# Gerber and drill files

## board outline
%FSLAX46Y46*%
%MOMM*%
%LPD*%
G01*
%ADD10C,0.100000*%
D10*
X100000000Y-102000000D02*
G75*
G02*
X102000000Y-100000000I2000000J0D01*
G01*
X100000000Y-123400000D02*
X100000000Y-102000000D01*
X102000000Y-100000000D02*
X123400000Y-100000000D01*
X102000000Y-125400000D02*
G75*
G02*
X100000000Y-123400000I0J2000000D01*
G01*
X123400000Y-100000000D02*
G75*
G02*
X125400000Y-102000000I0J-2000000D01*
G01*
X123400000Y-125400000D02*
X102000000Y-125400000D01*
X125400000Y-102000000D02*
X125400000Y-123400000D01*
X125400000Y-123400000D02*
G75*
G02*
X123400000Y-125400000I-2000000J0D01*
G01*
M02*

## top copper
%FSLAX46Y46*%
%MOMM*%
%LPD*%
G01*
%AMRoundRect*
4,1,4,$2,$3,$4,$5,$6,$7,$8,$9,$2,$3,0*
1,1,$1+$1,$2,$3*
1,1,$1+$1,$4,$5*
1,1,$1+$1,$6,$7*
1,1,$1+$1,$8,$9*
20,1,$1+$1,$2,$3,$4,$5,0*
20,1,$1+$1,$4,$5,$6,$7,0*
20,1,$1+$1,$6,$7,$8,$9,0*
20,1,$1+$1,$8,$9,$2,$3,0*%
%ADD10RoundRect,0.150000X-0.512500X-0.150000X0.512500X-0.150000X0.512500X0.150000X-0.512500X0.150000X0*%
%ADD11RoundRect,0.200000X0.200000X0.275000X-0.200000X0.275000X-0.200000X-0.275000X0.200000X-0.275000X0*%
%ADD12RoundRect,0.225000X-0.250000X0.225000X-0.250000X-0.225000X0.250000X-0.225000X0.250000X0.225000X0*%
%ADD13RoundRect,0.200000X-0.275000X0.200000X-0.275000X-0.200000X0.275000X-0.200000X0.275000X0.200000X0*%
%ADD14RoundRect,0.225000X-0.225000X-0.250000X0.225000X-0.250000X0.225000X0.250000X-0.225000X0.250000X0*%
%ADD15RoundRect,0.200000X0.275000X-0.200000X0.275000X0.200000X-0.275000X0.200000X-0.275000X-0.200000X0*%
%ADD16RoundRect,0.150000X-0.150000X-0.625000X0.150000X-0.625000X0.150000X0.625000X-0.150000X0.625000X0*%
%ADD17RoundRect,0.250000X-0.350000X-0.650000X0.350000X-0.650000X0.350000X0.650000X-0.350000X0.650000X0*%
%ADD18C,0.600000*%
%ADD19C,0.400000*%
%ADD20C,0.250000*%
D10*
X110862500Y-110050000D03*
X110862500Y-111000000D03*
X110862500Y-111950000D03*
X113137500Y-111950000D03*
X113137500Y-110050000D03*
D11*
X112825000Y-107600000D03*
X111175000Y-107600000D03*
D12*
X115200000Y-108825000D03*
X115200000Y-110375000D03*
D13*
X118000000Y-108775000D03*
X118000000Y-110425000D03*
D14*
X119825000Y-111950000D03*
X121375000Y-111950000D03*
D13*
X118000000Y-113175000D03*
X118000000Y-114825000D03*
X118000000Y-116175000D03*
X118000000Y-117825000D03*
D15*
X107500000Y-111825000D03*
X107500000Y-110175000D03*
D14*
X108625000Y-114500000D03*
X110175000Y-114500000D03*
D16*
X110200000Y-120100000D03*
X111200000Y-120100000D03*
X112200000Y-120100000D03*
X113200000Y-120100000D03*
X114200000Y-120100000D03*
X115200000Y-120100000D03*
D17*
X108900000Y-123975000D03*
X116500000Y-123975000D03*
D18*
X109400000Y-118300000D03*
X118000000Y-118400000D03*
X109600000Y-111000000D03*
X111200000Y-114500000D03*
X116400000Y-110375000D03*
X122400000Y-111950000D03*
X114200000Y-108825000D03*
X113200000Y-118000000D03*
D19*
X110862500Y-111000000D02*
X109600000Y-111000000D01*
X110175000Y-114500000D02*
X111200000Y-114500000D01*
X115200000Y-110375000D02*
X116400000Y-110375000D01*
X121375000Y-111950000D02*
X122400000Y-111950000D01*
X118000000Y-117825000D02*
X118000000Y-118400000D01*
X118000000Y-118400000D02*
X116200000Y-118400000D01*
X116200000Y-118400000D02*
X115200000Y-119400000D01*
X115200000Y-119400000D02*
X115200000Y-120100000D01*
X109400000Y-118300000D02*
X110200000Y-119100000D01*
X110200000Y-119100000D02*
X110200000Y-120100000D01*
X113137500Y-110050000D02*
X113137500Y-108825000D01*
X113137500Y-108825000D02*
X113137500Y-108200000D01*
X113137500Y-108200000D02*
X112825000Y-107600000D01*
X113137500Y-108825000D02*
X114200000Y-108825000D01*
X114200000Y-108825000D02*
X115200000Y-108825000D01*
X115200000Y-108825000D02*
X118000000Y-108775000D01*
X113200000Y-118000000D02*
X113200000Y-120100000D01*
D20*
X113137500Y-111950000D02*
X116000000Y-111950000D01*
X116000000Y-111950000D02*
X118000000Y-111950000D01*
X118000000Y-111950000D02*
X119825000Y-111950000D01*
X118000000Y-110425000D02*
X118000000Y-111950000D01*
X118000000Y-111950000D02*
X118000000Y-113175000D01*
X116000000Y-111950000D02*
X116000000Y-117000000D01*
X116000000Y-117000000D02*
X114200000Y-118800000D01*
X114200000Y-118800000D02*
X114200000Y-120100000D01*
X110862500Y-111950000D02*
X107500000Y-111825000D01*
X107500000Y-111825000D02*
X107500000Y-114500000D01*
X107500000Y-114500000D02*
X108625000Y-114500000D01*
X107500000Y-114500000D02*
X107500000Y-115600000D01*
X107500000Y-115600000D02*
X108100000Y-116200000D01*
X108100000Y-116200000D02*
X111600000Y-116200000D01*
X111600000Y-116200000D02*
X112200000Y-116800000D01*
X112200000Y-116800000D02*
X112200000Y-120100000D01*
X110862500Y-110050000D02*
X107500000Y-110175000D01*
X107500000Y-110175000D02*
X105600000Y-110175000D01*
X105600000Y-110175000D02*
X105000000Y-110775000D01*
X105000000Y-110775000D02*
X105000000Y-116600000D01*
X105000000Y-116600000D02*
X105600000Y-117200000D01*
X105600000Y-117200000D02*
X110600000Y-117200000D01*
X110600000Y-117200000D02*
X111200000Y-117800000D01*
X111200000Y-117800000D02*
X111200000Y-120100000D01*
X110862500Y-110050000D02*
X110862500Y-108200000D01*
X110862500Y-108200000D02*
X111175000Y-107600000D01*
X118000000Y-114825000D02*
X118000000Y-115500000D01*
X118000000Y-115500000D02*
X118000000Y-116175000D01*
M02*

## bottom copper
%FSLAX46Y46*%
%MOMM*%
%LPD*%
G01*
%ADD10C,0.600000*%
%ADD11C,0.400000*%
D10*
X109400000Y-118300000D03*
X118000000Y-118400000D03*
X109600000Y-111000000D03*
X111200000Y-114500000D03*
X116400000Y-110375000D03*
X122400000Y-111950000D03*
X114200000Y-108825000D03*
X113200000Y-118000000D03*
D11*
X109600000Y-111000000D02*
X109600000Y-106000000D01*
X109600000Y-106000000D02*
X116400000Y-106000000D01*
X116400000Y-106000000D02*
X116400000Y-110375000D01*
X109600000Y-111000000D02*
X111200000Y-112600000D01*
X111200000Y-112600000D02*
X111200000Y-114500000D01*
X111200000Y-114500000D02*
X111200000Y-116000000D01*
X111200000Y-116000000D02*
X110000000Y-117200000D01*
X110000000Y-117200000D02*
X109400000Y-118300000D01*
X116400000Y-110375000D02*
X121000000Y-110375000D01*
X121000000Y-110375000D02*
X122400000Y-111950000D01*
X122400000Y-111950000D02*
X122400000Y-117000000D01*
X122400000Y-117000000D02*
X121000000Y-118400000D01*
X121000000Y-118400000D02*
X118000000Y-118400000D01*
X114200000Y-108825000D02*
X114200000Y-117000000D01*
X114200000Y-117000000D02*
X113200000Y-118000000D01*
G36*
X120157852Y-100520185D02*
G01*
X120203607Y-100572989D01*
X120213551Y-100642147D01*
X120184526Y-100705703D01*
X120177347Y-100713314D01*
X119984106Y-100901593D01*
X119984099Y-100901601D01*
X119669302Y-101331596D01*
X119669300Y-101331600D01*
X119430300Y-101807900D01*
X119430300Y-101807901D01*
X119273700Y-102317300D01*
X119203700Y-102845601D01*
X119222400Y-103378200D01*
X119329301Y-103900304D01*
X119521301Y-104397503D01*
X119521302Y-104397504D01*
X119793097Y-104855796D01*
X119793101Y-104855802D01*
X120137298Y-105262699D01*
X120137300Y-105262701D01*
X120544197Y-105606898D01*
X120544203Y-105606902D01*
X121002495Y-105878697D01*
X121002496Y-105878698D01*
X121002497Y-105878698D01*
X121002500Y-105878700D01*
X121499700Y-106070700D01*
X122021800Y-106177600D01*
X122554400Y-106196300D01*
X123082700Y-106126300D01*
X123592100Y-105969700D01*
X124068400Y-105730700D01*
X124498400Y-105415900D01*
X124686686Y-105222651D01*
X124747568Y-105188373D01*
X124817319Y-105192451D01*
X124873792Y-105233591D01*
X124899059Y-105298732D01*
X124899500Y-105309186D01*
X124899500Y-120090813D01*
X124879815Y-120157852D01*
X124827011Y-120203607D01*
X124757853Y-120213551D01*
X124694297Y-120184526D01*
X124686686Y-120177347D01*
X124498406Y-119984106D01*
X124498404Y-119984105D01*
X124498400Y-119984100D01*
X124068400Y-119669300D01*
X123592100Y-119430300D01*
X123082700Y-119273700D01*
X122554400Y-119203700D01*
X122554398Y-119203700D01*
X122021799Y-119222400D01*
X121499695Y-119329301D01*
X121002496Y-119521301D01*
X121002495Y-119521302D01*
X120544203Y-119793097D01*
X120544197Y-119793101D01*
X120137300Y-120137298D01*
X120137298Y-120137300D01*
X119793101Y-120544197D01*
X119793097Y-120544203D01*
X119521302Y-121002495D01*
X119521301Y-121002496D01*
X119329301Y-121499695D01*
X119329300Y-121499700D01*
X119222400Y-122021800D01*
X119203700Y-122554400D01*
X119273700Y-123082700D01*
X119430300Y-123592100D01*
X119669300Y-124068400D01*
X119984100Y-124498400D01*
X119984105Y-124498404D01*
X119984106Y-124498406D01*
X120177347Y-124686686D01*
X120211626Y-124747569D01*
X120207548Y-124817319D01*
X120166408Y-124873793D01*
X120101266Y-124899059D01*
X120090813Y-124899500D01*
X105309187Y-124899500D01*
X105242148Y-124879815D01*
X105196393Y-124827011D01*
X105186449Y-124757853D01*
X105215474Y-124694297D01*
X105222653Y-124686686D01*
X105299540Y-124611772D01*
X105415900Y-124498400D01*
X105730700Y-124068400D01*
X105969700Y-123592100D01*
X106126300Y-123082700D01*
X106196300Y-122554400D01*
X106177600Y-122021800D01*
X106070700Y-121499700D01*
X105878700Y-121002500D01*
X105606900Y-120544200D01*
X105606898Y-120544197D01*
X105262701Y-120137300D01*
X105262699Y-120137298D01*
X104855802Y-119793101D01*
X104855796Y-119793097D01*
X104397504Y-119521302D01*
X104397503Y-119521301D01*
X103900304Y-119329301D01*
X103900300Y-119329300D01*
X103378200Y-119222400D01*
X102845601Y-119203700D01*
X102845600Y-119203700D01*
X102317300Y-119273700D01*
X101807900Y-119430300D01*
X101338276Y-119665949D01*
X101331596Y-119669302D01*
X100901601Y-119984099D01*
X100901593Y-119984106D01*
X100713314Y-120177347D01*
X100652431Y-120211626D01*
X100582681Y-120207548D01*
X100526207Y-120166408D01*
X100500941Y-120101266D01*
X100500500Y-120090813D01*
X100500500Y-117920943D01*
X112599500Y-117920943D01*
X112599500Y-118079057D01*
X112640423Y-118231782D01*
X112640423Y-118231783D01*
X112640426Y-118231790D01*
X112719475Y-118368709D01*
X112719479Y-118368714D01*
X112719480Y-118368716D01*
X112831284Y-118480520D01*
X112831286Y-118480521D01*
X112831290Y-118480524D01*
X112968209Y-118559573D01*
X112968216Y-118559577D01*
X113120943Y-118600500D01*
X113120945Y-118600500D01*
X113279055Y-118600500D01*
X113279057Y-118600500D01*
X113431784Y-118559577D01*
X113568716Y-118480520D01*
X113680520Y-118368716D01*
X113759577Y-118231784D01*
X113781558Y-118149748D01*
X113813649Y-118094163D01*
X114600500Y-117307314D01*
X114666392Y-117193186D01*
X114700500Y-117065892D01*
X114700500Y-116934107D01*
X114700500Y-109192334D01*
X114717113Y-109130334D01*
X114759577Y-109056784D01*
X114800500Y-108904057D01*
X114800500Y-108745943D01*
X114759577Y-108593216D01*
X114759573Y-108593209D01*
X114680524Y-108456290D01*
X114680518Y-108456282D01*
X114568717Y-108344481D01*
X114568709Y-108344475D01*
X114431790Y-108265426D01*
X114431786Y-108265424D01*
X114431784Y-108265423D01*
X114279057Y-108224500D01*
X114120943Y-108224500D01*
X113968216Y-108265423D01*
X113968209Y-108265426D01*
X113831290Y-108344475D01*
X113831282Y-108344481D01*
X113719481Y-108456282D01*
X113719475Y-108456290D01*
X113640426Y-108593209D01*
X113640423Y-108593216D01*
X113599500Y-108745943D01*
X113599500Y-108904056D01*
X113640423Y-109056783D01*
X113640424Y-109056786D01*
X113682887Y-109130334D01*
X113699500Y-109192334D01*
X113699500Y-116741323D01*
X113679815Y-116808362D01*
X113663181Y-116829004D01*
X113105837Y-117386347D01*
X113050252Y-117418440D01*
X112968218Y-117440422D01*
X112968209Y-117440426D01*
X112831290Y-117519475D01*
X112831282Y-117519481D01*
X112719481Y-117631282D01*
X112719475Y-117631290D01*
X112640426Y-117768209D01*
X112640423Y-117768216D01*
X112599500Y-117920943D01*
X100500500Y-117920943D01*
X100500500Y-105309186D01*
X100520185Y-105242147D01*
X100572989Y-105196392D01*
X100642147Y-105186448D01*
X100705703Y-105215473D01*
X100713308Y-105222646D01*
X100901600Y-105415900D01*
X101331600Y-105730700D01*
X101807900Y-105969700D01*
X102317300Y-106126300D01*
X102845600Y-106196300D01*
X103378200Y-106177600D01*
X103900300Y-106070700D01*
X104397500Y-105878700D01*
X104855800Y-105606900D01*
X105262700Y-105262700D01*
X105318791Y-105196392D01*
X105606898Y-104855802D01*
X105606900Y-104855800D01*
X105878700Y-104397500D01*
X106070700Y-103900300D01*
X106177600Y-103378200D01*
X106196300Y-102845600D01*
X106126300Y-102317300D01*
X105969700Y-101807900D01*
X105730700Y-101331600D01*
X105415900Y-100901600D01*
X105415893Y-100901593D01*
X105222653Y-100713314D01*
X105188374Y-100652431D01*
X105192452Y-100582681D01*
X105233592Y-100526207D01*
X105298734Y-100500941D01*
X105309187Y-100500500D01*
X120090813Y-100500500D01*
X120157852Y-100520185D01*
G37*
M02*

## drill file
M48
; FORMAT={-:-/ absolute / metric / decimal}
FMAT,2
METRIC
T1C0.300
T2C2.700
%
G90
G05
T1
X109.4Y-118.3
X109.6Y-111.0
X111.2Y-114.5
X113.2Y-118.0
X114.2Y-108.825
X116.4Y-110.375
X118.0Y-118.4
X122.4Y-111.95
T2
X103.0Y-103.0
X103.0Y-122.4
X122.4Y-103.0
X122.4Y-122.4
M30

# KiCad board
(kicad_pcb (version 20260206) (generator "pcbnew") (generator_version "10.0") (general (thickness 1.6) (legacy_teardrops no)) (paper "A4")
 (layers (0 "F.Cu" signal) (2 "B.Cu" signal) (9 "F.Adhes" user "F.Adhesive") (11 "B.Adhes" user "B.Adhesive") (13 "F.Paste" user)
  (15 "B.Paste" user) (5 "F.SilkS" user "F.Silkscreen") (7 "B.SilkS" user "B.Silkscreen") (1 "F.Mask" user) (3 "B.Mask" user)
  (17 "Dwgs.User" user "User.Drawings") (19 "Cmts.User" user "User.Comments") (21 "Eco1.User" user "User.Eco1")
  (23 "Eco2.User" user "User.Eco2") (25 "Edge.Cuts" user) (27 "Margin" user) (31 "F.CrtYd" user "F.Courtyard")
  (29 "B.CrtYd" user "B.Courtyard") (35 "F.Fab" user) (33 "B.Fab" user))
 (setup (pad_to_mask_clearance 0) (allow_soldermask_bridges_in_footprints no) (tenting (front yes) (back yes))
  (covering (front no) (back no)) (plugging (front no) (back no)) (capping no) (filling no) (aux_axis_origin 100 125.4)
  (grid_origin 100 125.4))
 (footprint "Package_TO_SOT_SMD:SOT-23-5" (layer "F.Cu") (at 112 111)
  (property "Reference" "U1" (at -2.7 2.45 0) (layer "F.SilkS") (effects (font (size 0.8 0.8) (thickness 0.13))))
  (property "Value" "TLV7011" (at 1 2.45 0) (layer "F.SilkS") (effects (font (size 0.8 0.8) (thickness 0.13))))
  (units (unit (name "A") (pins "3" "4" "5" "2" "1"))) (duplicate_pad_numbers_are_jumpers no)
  (pad "1" smd roundrect (at -1.1375 -0.95) (size 1.325 0.6) (layers "F.Cu" "F.Mask" "F.Paste") (roundrect_rratio 0.25)
   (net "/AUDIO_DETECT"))
  (pad "2" smd roundrect (at -1.1375 0) (size 1.325 0.6) (layers "F.Cu" "F.Mask" "F.Paste") (roundrect_rratio 0.25) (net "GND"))
  (pad "3" smd roundrect (at -1.1375 0.95) (size 1.325 0.6) (layers "F.Cu" "F.Mask" "F.Paste") (roundrect_rratio 0.25)
   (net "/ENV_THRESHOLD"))
  (pad "4" smd roundrect (at 1.1375 0.95) (size 1.325 0.6) (layers "F.Cu" "F.Mask" "F.Paste") (roundrect_rratio 0.25) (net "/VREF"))
  (pad "5" smd roundrect (at 1.1375 -0.95) (size 1.325 0.6) (layers "F.Cu" "F.Mask" "F.Paste") (roundrect_rratio 0.25) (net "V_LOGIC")))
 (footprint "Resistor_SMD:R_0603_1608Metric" (layer "F.Cu") (at 112 107.6 180)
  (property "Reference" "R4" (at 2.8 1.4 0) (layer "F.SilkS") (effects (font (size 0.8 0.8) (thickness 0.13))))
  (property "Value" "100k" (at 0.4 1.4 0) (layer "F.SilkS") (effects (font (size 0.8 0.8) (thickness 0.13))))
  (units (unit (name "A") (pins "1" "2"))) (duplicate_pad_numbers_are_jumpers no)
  (pad "1" smd roundrect (at -0.825 0 180) (size 0.8 0.95) (layers "F.Cu" "F.Mask" "F.Paste") (roundrect_rratio 0.25) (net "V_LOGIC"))
  (pad "2" smd roundrect (at 0.825 0 180) (size 0.8 0.95) (layers "F.Cu" "F.Mask" "F.Paste") (roundrect_rratio 0.25) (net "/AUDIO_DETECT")))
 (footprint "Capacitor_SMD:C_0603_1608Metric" (layer "F.Cu") (at 115.2 109.6 -90)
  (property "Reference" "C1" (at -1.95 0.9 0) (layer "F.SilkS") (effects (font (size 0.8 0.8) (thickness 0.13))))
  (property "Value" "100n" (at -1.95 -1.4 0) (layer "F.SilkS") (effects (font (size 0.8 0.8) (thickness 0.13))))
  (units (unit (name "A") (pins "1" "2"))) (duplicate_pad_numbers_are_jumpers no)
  (pad "1" smd roundrect (at -0.775 0 270) (size 0.9 0.95) (layers "F.Cu" "F.Mask" "F.Paste") (roundrect_rratio 0.25) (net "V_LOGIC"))
  (pad "2" smd roundrect (at 0.775 0 270) (size 0.9 0.95) (layers "F.Cu" "F.Mask" "F.Paste") (roundrect_rratio 0.25) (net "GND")))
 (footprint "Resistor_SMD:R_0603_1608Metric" (layer "F.Cu") (at 118 109.6 -90)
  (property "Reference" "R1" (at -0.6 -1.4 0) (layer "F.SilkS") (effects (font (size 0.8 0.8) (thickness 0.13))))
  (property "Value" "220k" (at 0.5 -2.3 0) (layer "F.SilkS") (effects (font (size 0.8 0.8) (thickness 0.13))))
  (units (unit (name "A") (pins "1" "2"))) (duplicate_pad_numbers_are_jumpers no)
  (pad "1" smd roundrect (at -0.825 0 270) (size 0.8 0.95) (layers "F.Cu" "F.Mask" "F.Paste") (roundrect_rratio 0.25) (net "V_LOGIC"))
  (pad "2" smd roundrect (at 0.825 0 270) (size 0.8 0.95) (layers "F.Cu" "F.Mask" "F.Paste") (roundrect_rratio 0.25) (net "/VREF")))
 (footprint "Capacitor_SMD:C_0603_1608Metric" (layer "F.Cu") (at 120.6 111.95)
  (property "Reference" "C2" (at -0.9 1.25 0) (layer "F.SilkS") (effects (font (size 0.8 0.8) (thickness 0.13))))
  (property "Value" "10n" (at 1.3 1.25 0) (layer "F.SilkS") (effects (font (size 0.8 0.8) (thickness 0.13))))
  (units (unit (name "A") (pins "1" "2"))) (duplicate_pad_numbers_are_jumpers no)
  (pad "1" smd roundrect (at -0.775 0) (size 0.9 0.95) (layers "F.Cu" "F.Mask" "F.Paste") (roundrect_rratio 0.25) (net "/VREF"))
  (pad "2" smd roundrect (at 0.775 0) (size 0.9 0.95) (layers "F.Cu" "F.Mask" "F.Paste") (roundrect_rratio 0.25) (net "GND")))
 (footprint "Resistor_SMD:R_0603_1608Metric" (layer "F.Cu") (at 118 114 -90)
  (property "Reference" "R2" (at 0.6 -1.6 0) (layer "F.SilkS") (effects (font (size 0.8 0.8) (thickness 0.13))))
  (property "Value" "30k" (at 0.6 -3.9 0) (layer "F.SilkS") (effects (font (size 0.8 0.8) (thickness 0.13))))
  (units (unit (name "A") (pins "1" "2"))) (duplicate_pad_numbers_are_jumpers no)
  (pad "1" smd roundrect (at -0.825 0 270) (size 0.8 0.95) (layers "F.Cu" "F.Mask" "F.Paste") (roundrect_rratio 0.25) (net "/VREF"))
  (pad "2" smd roundrect (at 0.825 0 270) (size 0.8 0.95) (layers "F.Cu" "F.Mask" "F.Paste") (roundrect_rratio 0.25) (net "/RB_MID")))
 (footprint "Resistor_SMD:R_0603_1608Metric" (layer "F.Cu") (at 118 117 -90)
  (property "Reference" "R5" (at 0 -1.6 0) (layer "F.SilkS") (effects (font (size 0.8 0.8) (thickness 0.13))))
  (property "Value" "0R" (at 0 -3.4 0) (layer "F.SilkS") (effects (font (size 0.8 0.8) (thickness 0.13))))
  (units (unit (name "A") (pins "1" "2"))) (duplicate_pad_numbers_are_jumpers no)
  (pad "1" smd roundrect (at -0.825 0 270) (size 0.8 0.95) (layers "F.Cu" "F.Mask" "F.Paste") (roundrect_rratio 0.25) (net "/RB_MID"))
  (pad "2" smd roundrect (at 0.825 0 270) (size 0.8 0.95) (layers "F.Cu" "F.Mask" "F.Paste") (roundrect_rratio 0.25) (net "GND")))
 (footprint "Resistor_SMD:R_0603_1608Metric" (layer "F.Cu") (at 107.5 111 90)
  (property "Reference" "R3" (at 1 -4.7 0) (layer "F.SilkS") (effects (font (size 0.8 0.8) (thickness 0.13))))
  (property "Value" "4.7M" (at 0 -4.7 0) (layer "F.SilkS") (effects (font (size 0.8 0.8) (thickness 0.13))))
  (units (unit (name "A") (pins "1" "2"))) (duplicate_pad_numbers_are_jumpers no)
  (pad "1" smd roundrect (at -0.825 0 90) (size 0.8 0.95) (layers "F.Cu" "F.Mask" "F.Paste") (roundrect_rratio 0.25) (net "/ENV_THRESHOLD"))
  (pad "2" smd roundrect (at 0.825 0 90) (size 0.8 0.95) (layers "F.Cu" "F.Mask" "F.Paste") (roundrect_rratio 0.25) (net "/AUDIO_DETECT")))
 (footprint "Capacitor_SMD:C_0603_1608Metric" (layer "F.Cu") (at 109.4 114.5)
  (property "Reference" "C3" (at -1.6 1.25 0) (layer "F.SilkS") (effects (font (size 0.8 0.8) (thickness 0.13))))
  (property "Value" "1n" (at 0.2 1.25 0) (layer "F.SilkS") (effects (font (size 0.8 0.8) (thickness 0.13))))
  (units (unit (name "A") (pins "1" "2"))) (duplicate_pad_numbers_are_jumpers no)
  (pad "1" smd roundrect (at -0.775 0) (size 0.9 0.95) (layers "F.Cu" "F.Mask" "F.Paste") (roundrect_rratio 0.25) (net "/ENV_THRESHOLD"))
  (pad "2" smd roundrect (at 0.775 0) (size 0.9 0.95) (layers "F.Cu" "F.Mask" "F.Paste") (roundrect_rratio 0.25) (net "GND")))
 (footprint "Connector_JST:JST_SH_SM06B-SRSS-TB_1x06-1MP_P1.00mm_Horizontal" (layer "F.Cu") (at 112.7 122.1)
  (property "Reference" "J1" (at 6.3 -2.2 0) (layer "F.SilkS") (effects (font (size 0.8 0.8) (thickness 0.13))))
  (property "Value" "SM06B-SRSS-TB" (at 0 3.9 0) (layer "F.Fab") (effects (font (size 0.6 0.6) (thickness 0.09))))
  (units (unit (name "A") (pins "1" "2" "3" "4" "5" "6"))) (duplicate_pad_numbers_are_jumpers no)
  (pad "1" smd roundrect (at -2.5 -2) (size 0.6 1.55) (layers "F.Cu" "F.Mask" "F.Paste") (roundrect_rratio 0.25) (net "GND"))
  (pad "2" smd roundrect (at -1.5 -2) (size 0.6 1.55) (layers "F.Cu" "F.Mask" "F.Paste") (roundrect_rratio 0.25) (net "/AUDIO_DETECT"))
  (pad "3" smd roundrect (at -0.5 -2) (size 0.6 1.55) (layers "F.Cu" "F.Mask" "F.Paste") (roundrect_rratio 0.25) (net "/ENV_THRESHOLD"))
  (pad "4" smd roundrect (at 0.5 -2) (size 0.6 1.55) (layers "F.Cu" "F.Mask" "F.Paste") (roundrect_rratio 0.25) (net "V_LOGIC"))
  (pad "5" smd roundrect (at 1.5 -2) (size 0.6 1.55) (layers "F.Cu" "F.Mask" "F.Paste") (roundrect_rratio 0.25) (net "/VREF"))
  (pad "6" smd roundrect (at 2.5 -2) (size 0.6 1.55) (layers "F.Cu" "F.Mask" "F.Paste") (roundrect_rratio 0.25) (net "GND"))
  (pad "MP" smd roundrect (at -3.8 1.875) (size 1.2 1.8) (layers "F.Cu" "F.Mask" "F.Paste") (roundrect_rratio 0.208333))
  (pad "MP" smd roundrect (at 3.8 1.875) (size 1.2 1.8) (layers "F.Cu" "F.Mask" "F.Paste") (roundrect_rratio 0.208333)))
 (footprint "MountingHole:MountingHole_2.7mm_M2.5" (layer "F.Cu") (at 103 103)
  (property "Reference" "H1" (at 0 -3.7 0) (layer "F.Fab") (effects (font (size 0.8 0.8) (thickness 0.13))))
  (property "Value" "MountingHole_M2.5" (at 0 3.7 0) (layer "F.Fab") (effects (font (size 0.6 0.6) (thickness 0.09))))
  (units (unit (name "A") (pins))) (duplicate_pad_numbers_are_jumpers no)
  (pad "" np_thru_hole circle (at 0 0) (size 2.7 2.7) (drill 2.7) (layers "*.Cu" "*.Mask")))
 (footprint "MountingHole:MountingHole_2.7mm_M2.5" (layer "F.Cu") (at 122.4 103)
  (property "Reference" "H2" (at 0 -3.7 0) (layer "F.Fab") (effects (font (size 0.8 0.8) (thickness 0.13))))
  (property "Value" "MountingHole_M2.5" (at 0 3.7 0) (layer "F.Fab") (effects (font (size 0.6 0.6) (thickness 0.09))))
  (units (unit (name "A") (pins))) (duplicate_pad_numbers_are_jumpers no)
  (pad "" np_thru_hole circle (at 0 0) (size 2.7 2.7) (drill 2.7) (layers "*.Cu" "*.Mask")))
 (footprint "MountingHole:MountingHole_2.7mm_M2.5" (layer "F.Cu") (at 103 122.4)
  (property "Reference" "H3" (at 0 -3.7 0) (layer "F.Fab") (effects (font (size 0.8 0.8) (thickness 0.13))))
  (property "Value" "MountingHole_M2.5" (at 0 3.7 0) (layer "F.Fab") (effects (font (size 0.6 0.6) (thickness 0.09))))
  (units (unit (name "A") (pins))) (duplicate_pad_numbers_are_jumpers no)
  (pad "" np_thru_hole circle (at 0 0) (size 2.7 2.7) (drill 2.7) (layers "*.Cu" "*.Mask")))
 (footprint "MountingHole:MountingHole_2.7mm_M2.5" (layer "F.Cu") (at 122.4 122.4)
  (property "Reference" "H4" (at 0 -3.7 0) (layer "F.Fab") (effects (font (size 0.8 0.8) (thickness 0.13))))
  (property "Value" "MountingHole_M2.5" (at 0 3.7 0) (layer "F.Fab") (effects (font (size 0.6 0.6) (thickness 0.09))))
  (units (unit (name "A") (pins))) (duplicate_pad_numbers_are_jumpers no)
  (pad "" np_thru_hole circle (at 0 0) (size 2.7 2.7) (drill 2.7) (layers "*.Cu" "*.Mask")))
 (gr_arc (start 100 102) (mid 100.5858 100.5858) (end 102 100) (stroke (width 0.1) (type default)) (layer "Edge.Cuts"))
 (gr_line (start 100 123.4) (end 100 102) (stroke (width 0.1) (type default)) (layer "Edge.Cuts"))
 (gr_line (start 102 100) (end 123.4 100) (stroke (width 0.1) (type default)) (layer "Edge.Cuts"))
 (gr_arc (start 102 125.4) (mid 100.5858 124.8142) (end 100 123.4) (stroke (width 0.1) (type default)) (layer "Edge.Cuts"))
 (gr_arc (start 123.4 100) (mid 124.8142 100.5858) (end 125.4 102) (stroke (width 0.1) (type default)) (layer "Edge.Cuts"))
 (gr_line (start 123.4 125.4) (end 102 125.4) (stroke (width 0.1) (type default)) (layer "Edge.Cuts"))
 (gr_line (start 125.4 102) (end 125.4 123.4) (stroke (width 0.1) (type default)) (layer "Edge.Cuts"))
 (gr_arc (start 125.4 123.4) (mid 124.8142 124.8142) (end 123.4 125.4) (stroke (width 0.1) (type default)) (layer "Edge.Cuts"))
 (segment (start 110.8625 111) (end 109.6 111) (width 0.4) (layer "F.Cu") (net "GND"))
 (segment (start 110.175 114.5) (end 111.2 114.5) (width 0.4) (layer "F.Cu") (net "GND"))
 (segment (start 115.2 110.375) (end 116.4 110.375) (width 0.4) (layer "F.Cu") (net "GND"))
 (segment (start 121.375 111.95) (end 122.4 111.95) (width 0.4) (layer "F.Cu") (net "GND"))
 (segment (start 118 117.825) (end 118 118.4) (width 0.4) (layer "F.Cu") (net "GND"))
 (segment (start 118 118.4) (end 116.2 118.4) (width 0.4) (layer "F.Cu") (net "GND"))
 (segment (start 116.2 118.4) (end 115.2 119.4) (width 0.4) (layer "F.Cu") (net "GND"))
 (segment (start 115.2 119.4) (end 115.2 120.1) (width 0.4) (layer "F.Cu") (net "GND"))
 (segment (start 109.4 118.3) (end 110.2 119.1) (width 0.4) (layer "F.Cu") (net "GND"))
 (segment (start 110.2 119.1) (end 110.2 120.1) (width 0.4) (layer "F.Cu") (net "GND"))
 (via (at 109.4 118.3) (size 0.6) (drill 0.3) (layers "F.Cu" "B.Cu") (capping no) (covering (front no) (back no))
  (plugging (front no) (back no)) (filling no) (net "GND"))
 (via (at 118 118.4) (size 0.6) (drill 0.3) (layers "F.Cu" "B.Cu") (capping no) (covering (front no) (back no))
  (plugging (front no) (back no)) (filling no) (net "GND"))
 (via (at 109.6 111) (size 0.6) (drill 0.3) (layers "F.Cu" "B.Cu") (capping no) (covering (front no) (back no))
  (plugging (front no) (back no)) (filling no) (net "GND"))
 (via (at 111.2 114.5) (size 0.6) (drill 0.3) (layers "F.Cu" "B.Cu") (capping no) (covering (front no) (back no))
  (plugging (front no) (back no)) (filling no) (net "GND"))
 (via (at 116.4 110.375) (size 0.6) (drill 0.3) (layers "F.Cu" "B.Cu") (capping no) (covering (front no) (back no))
  (plugging (front no) (back no)) (filling no) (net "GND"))
 (via (at 122.4 111.95) (size 0.6) (drill 0.3) (layers "F.Cu" "B.Cu") (capping no) (covering (front no) (back no))
  (plugging (front no) (back no)) (filling no) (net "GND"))
 (segment (start 109.6 111) (end 109.6 106) (width 0.4) (layer "B.Cu") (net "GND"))
 (segment (start 109.6 106) (end 116.4 106) (width 0.4) (layer "B.Cu") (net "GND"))
 (segment (start 116.4 106) (end 116.4 110.375) (width 0.4) (layer "B.Cu") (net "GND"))
 (segment (start 109.6 111) (end 111.2 112.6) (width 0.4) (layer "B.Cu") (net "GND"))
 (segment (start 111.2 112.6) (end 111.2 114.5) (width 0.4) (layer "B.Cu") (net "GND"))
 (segment (start 111.2 114.5) (end 111.2 116) (width 0.4) (layer "B.Cu") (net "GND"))
 (segment (start 111.2 116) (end 110 117.2) (width 0.4) (layer "B.Cu") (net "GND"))
 (segment (start 110 117.2) (end 109.4 118.3) (width 0.4) (layer "B.Cu") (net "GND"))
 (segment (start 116.4 110.375) (end 121 110.375) (width 0.4) (layer "B.Cu") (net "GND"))
 (segment (start 121 110.375) (end 122.4 111.95) (width 0.4) (layer "B.Cu") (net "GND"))
 (segment (start 122.4 111.95) (end 122.4 117) (width 0.4) (layer "B.Cu") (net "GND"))
 (segment (start 122.4 117) (end 121 118.4) (width 0.4) (layer "B.Cu") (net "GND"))
 (segment (start 121 118.4) (end 118 118.4) (width 0.4) (layer "B.Cu") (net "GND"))
 (segment (start 113.1375 110.05) (end 113.1375 108.825) (width 0.4) (layer "F.Cu") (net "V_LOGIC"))
 (segment (start 113.1375 108.825) (end 113.1375 108.2) (width 0.4) (layer "F.Cu") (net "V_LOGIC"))
 (segment (start 113.1375 108.2) (end 112.825 107.6) (width 0.4) (layer "F.Cu") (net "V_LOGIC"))
 (segment (start 113.1375 108.825) (end 114.2 108.825) (width 0.4) (layer "F.Cu") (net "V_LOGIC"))
 (segment (start 114.2 108.825) (end 115.2 108.825) (width 0.4) (layer "F.Cu") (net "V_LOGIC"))
 (segment (start 115.2 108.825) (end 118 108.775) (width 0.4) (layer "F.Cu") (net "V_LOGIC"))
 (segment (start 113.2 118) (end 113.2 120.1) (width 0.4) (layer "F.Cu") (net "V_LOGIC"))
 (via (at 114.2 108.825) (size 0.6) (drill 0.3) (layers "F.Cu" "B.Cu") (capping no) (covering (front no) (back no))
  (plugging (front no) (back no)) (filling no) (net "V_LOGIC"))
 (via (at 113.2 118) (size 0.6) (drill 0.3) (layers "F.Cu" "B.Cu") (capping no) (covering (front no) (back no))
  (plugging (front no) (back no)) (filling no) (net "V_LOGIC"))
 (segment (start 114.2 108.825) (end 114.2 117) (width 0.4) (layer "B.Cu") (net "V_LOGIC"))
 (segment (start 114.2 117) (end 113.2 118) (width 0.4) (layer "B.Cu") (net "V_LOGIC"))
 (segment (start 113.1375 111.95) (end 116 111.95) (width 0.25) (layer "F.Cu") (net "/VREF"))
 (segment (start 116 111.95) (end 118 111.95) (width 0.25) (layer "F.Cu") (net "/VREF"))
 (segment (start 118 111.95) (end 119.825 111.95) (width 0.25) (layer "F.Cu") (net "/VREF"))
 (segment (start 118 110.425) (end 118 111.95) (width 0.25) (layer "F.Cu") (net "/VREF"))
 (segment (start 118 111.95) (end 118 113.175) (width 0.25) (layer "F.Cu") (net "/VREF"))
 (segment (start 116 111.95) (end 116 117) (width 0.25) (layer "F.Cu") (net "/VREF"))
 (segment (start 116 117) (end 114.2 118.8) (width 0.25) (layer "F.Cu") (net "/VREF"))
 (segment (start 114.2 118.8) (end 114.2 120.1) (width 0.25) (layer "F.Cu") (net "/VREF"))
 (segment (start 110.8625 111.95) (end 107.5 111.825) (width 0.25) (layer "F.Cu") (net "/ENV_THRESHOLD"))
 (segment (start 107.5 111.825) (end 107.5 114.5) (width 0.25) (layer "F.Cu") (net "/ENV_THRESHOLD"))
 (segment (start 107.5 114.5) (end 108.625 114.5) (width 0.25) (layer "F.Cu") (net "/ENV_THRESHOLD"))
 (segment (start 107.5 114.5) (end 107.5 115.6) (width 0.25) (layer "F.Cu") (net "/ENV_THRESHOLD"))
 (segment (start 107.5 115.6) (end 108.1 116.2) (width 0.25) (layer "F.Cu") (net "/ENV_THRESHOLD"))
 (segment (start 108.1 116.2) (end 111.6 116.2) (width 0.25) (layer "F.Cu") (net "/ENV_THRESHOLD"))
 (segment (start 111.6 116.2) (end 112.2 116.8) (width 0.25) (layer "F.Cu") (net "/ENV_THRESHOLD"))
 (segment (start 112.2 116.8) (end 112.2 120.1) (width 0.25) (layer "F.Cu") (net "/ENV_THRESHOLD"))
 (segment (start 110.8625 110.05) (end 107.5 110.175) (width 0.25) (layer "F.Cu") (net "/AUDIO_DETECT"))
 (segment (start 107.5 110.175) (end 105.6 110.175) (width 0.25) (layer "F.Cu") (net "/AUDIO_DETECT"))
 (segment (start 105.6 110.175) (end 105 110.775) (width 0.25) (layer "F.Cu") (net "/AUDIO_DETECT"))
 (segment (start 105 110.775) (end 105 116.6) (width 0.25) (layer "F.Cu") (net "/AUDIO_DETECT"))
 (segment (start 105 116.6) (end 105.6 117.2) (width 0.25) (layer "F.Cu") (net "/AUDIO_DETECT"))
 (segment (start 105.6 117.2) (end 110.6 117.2) (width 0.25) (layer "F.Cu") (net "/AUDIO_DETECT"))
 (segment (start 110.6 117.2) (end 111.2 117.8) (width 0.25) (layer "F.Cu") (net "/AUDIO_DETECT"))
 (segment (start 111.2 117.8) (end 111.2 120.1) (width 0.25) (layer "F.Cu") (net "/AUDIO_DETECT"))
 (segment (start 110.8625 110.05) (end 110.8625 108.2) (width 0.25) (layer "F.Cu") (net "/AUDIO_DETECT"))
 (segment (start 110.8625 108.2) (end 111.175 107.6) (width 0.25) (layer "F.Cu") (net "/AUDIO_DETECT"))
 (segment (start 118 114.825) (end 118 115.5) (width 0.25) (layer "F.Cu") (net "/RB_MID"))
 (segment (start 118 115.5) (end 118 116.175) (width 0.25) (layer "F.Cu") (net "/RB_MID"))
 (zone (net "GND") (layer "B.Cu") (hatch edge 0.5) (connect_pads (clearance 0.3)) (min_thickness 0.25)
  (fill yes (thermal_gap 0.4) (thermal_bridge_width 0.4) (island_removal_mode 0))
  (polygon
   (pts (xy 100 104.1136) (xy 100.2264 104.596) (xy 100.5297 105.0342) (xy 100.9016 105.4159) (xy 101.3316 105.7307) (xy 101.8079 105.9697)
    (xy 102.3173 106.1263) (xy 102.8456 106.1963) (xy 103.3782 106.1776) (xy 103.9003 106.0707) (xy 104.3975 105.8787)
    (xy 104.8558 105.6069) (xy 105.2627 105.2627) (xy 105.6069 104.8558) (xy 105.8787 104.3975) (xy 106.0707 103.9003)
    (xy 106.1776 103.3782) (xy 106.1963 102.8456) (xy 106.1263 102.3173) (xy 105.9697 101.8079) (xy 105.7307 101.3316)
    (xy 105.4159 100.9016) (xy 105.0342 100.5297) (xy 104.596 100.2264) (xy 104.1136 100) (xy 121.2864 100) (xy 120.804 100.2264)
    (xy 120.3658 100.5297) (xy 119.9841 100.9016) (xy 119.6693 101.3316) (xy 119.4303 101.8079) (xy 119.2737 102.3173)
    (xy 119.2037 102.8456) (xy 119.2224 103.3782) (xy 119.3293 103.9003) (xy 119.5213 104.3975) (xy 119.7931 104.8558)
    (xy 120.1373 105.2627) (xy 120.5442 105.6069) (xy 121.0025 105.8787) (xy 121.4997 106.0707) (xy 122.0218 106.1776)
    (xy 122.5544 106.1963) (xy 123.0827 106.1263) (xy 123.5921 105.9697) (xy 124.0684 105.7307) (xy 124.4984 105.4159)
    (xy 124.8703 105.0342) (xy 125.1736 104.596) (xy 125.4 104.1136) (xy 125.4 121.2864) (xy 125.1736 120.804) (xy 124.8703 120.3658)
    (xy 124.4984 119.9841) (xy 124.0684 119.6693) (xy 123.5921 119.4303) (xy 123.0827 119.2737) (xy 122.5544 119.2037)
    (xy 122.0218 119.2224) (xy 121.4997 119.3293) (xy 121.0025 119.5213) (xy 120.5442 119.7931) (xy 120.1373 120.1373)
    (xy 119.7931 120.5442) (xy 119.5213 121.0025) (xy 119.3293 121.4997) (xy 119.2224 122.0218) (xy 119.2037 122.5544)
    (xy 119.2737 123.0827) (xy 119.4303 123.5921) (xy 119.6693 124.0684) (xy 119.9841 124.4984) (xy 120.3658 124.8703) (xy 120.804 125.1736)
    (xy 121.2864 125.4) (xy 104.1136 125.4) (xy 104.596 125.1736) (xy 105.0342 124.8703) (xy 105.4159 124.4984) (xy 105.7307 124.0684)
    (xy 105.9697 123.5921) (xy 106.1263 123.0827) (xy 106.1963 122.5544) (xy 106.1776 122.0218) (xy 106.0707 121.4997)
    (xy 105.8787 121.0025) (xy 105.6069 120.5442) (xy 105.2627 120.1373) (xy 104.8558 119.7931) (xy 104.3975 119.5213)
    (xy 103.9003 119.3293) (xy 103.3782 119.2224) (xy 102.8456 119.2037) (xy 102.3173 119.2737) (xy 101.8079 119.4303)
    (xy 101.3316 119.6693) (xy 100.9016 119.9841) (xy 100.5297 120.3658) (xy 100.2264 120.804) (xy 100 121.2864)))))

